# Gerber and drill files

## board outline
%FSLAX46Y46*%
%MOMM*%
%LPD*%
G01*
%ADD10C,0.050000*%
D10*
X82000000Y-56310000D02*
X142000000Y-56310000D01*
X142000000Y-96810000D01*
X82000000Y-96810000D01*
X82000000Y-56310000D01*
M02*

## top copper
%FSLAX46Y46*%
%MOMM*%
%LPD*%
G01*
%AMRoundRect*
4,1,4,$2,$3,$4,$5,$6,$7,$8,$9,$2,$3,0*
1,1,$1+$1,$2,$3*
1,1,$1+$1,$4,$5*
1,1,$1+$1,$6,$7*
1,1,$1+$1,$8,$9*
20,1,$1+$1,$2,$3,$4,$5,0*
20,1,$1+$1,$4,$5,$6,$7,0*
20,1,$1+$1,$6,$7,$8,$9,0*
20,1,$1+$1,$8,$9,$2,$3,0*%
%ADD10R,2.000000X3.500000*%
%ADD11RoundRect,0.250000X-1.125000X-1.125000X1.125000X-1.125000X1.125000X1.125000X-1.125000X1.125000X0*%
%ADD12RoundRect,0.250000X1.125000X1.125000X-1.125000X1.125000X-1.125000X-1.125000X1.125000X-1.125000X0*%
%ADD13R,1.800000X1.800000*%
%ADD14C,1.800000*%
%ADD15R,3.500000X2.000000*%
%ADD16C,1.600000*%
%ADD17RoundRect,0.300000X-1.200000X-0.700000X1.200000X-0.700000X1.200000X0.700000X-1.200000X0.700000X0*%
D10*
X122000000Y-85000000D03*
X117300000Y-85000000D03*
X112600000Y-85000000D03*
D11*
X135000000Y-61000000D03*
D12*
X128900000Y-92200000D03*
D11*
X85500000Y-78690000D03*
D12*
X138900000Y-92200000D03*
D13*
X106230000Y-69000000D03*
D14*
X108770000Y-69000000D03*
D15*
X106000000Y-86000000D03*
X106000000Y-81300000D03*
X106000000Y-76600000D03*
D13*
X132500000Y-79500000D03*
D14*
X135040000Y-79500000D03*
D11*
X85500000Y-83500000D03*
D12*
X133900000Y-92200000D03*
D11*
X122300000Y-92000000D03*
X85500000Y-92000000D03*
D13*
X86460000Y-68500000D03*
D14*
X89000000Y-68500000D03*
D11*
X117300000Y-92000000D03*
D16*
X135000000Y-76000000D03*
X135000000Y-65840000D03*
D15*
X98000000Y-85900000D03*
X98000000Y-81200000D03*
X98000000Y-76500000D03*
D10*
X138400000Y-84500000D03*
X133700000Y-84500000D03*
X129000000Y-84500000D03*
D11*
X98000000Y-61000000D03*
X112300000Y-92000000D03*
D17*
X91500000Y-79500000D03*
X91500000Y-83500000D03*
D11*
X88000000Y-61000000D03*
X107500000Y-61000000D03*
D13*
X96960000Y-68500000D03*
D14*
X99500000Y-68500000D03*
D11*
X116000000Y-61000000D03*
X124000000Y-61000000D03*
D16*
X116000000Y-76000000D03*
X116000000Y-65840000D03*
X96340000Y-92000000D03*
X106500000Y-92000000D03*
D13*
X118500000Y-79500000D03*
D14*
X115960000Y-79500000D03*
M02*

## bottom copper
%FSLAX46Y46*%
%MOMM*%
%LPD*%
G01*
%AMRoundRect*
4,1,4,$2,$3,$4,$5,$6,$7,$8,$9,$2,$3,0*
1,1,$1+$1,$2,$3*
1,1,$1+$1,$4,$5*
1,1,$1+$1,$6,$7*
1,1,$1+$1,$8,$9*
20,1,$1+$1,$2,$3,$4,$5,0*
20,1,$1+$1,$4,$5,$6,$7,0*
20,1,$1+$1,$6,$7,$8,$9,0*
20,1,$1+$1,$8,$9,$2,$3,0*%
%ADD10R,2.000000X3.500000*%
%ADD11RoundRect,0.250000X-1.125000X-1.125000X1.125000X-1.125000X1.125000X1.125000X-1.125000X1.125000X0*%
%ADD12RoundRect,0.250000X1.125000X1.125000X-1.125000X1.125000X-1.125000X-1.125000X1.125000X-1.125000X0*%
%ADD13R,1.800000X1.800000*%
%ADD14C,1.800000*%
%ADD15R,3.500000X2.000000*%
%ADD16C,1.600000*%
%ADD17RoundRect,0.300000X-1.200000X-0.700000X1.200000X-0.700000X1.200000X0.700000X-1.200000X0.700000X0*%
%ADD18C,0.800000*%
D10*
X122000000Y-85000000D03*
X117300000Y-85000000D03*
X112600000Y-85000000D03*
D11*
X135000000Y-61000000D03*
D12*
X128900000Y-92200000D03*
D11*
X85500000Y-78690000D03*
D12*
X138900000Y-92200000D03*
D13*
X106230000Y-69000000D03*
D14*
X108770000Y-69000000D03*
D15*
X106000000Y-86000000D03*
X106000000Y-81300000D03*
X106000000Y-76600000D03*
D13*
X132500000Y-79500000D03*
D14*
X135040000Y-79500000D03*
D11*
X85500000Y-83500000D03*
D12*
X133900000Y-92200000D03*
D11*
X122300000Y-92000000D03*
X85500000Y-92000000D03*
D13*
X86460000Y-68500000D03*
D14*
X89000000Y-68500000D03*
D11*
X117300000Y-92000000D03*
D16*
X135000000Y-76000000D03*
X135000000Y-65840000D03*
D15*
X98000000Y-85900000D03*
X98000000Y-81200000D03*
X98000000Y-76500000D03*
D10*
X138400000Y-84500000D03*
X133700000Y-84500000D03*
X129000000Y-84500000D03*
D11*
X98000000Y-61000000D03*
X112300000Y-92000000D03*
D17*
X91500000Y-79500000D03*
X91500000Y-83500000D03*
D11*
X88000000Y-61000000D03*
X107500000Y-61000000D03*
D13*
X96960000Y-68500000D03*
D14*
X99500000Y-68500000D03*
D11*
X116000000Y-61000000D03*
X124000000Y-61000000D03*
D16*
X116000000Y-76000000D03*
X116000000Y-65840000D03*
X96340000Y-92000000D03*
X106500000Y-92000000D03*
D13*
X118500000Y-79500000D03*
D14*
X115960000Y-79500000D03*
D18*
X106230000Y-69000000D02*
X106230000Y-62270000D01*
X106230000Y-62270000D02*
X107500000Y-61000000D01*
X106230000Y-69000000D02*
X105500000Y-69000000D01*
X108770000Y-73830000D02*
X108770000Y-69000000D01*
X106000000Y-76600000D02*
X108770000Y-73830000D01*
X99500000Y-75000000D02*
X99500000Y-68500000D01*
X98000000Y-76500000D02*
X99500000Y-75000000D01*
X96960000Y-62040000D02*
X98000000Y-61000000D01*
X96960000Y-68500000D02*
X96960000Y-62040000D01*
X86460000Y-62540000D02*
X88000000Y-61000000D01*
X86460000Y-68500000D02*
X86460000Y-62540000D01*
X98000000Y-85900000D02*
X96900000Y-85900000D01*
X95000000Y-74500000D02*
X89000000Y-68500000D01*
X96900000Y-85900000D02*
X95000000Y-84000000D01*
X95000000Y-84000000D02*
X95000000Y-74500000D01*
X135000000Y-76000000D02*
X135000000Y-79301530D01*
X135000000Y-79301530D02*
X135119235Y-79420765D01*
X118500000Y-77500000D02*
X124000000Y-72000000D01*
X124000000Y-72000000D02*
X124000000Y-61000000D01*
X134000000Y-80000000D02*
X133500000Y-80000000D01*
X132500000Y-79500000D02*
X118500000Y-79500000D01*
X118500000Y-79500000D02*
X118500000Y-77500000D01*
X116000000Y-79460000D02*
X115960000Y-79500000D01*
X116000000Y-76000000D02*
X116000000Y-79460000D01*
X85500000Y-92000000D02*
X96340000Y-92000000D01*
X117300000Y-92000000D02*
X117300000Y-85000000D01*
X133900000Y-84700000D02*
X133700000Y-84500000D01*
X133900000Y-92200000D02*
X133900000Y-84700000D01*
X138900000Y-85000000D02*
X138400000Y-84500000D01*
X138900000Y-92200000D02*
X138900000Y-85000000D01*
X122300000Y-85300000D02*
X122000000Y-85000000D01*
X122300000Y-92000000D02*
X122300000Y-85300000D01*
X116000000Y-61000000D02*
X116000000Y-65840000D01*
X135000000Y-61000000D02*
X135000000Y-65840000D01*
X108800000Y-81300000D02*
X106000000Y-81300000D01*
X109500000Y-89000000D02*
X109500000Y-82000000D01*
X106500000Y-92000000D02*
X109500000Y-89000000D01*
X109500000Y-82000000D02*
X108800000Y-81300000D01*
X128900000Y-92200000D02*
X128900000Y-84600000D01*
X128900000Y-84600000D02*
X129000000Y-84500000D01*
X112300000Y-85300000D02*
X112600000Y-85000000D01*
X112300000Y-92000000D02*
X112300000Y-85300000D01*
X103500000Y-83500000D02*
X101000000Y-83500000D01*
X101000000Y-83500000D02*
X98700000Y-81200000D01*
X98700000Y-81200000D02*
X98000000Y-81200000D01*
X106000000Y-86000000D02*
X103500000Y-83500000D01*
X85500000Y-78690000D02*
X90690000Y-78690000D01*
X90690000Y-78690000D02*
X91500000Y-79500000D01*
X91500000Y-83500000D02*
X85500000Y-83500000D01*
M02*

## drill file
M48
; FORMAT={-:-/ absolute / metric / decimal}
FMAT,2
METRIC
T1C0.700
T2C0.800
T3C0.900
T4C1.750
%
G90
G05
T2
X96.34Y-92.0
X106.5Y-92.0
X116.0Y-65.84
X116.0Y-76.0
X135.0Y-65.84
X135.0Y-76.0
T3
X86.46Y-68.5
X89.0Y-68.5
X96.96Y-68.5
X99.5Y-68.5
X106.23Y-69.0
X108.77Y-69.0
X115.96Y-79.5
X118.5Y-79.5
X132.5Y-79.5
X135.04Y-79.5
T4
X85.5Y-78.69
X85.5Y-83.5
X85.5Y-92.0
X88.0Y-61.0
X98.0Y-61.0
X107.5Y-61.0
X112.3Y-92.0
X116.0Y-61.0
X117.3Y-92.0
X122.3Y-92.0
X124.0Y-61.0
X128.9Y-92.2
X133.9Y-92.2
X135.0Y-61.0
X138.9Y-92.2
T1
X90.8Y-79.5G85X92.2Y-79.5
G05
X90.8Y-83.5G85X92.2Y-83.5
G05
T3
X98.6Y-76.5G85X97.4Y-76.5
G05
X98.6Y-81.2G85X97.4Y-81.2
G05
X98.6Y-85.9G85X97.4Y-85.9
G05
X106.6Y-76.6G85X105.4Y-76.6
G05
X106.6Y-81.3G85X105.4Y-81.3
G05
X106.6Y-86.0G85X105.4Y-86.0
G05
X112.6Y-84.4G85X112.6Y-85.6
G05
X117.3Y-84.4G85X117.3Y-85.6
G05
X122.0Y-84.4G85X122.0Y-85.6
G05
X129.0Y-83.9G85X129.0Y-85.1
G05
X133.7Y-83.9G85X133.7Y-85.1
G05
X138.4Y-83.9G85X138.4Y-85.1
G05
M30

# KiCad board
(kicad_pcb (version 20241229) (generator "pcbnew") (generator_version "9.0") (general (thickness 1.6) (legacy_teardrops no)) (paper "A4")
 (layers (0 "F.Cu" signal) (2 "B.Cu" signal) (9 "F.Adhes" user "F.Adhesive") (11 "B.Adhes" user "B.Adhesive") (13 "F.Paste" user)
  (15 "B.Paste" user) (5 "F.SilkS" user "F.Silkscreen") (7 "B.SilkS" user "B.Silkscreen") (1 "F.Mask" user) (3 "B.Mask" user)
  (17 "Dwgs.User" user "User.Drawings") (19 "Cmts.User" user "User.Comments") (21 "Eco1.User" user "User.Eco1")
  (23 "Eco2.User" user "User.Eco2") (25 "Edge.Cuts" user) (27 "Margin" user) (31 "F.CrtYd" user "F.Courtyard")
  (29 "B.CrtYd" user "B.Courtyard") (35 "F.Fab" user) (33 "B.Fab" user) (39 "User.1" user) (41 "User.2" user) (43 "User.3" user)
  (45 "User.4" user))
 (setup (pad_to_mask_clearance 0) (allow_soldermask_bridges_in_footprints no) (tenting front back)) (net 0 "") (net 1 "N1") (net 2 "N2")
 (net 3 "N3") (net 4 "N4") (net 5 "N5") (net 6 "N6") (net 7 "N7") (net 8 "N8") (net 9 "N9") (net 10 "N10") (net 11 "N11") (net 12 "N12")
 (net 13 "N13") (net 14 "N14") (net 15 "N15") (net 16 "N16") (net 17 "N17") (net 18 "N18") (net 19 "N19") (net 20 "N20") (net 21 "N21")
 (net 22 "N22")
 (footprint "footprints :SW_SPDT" (layer "F.Cu") (at 117.3 85 -90)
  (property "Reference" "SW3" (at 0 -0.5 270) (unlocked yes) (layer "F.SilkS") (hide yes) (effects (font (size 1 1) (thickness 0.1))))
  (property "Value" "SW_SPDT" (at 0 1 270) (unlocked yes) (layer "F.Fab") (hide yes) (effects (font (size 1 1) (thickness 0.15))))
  (pad "1" thru_hole rect (at 0 -4.7 270) (size 3.5 2) (drill oval 2.1 0.9) (layers "*.Cu" "*.Mask") (remove_unused_layers no) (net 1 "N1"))
  (pad "2" thru_hole rect (at 0 0 270) (size 3.5 2) (drill oval 2.1 0.9) (layers "*.Cu" "*.Mask") (remove_unused_layers no) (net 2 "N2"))
  (pad "3" thru_hole rect (at 0 4.7 270) (size 3.5 2) (drill oval 2.1 0.9) (layers "*.Cu" "*.Mask") (remove_unused_layers no) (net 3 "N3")))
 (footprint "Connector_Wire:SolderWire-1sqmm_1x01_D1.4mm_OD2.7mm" (layer "F.Cu") (at 135 61)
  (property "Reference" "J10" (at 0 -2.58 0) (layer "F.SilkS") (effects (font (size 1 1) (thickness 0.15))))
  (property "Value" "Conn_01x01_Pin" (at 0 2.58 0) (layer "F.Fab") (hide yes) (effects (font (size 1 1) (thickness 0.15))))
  (pad "1" thru_hole roundrect (at 0 0) (size 2.75 2.75) (drill 1.75) (layers "*.Cu" "*.Mask") (remove_unused_layers no)
   (roundrect_rratio 0.090909) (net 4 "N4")))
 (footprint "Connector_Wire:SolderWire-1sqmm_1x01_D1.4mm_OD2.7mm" (layer "F.Cu") (at 128.9 92.2 180)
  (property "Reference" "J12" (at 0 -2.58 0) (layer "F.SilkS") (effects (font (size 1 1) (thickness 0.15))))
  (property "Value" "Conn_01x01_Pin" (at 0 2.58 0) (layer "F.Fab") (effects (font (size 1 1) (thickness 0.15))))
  (pad "1" thru_hole roundrect (at 0 0 180) (size 2.75 2.75) (drill 1.75) (layers "*.Cu" "*.Mask") (remove_unused_layers no)
   (roundrect_rratio 0.090909) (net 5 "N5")))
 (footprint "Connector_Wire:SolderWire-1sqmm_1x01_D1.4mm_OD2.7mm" (layer "F.Cu") (at 85.5 78.69)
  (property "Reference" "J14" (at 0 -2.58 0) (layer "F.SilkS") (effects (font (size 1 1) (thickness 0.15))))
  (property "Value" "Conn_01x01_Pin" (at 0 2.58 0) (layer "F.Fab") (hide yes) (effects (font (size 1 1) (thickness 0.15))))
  (pad "1" thru_hole roundrect (at 0 0) (size 2.75 2.75) (drill 1.75) (layers "*.Cu" "*.Mask") (remove_unused_layers no)
   (roundrect_rratio 0.090909) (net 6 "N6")))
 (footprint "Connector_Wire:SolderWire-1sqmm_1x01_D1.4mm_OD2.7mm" (layer "F.Cu") (at 138.9 92.2 180)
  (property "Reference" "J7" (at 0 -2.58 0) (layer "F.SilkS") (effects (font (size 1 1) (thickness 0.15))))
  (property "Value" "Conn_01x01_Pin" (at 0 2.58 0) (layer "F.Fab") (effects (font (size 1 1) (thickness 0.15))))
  (pad "1" thru_hole roundrect (at 0 0 180) (size 2.75 2.75) (drill 1.75) (layers "*.Cu" "*.Mask") (remove_unused_layers no)
   (roundrect_rratio 0.090909) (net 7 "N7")))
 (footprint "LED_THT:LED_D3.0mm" (layer "F.Cu") (at 106.23 69)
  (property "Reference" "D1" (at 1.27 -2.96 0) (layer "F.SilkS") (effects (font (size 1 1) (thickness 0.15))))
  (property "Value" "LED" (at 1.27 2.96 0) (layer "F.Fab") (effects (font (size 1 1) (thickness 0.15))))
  (pad "1" thru_hole rect (at 0 0) (size 1.8 1.8) (drill 0.9) (layers "*.Cu" "*.Mask") (remove_unused_layers no) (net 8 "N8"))
  (pad "2" thru_hole circle (at 2.54 0) (size 1.8 1.8) (drill 0.9) (layers "*.Cu" "*.Mask") (remove_unused_layers no) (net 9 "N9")))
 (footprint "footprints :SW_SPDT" (layer "F.Cu") (at 106 81.3 180)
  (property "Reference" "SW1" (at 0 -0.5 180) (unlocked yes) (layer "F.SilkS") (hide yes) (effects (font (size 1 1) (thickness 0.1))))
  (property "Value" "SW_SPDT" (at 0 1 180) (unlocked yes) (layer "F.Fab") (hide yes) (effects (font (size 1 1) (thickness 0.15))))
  (pad "1" thru_hole rect (at 0 -4.7 180) (size 3.5 2) (drill oval 2.1 0.9) (layers "*.Cu" "*.Mask") (remove_unused_layers no)
   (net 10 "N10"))
  (pad "2" thru_hole rect (at 0 0 180) (size 3.5 2) (drill oval 2.1 0.9) (layers "*.Cu" "*.Mask") (remove_unused_layers no) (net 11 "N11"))
  (pad "3" thru_hole rect (at 0 4.7 180) (size 3.5 2) (drill oval 2.1 0.9) (layers "*.Cu" "*.Mask") (remove_unused_layers no) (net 9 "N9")))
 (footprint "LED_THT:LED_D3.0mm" (layer "F.Cu") (at 132.5 79.5)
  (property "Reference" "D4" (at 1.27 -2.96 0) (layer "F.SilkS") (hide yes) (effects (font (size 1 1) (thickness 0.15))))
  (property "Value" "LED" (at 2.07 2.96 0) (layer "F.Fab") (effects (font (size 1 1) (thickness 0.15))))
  (pad "1" thru_hole rect (at 0 0) (size 1.8 1.8) (drill 0.9) (layers "*.Cu" "*.Mask") (remove_unused_layers no) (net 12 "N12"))
  (pad "2" thru_hole circle (at 2.54 0) (size 1.8 1.8) (drill 0.9) (layers "*.Cu" "*.Mask") (remove_unused_layers no) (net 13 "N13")))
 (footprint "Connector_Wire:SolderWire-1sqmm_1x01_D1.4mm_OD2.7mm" (layer "F.Cu") (at 85.5 83.5)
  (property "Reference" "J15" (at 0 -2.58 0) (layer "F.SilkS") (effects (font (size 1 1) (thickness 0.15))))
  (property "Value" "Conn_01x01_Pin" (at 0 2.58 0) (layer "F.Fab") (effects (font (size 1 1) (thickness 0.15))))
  (pad "1" thru_hole roundrect (at 0 0) (size 2.75 2.75) (drill 1.75) (layers "*.Cu" "*.Mask") (remove_unused_layers no)
   (roundrect_rratio 0.090909) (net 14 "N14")))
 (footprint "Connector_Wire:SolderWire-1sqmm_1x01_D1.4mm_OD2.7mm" (layer "F.Cu") (at 133.9 92.2 180)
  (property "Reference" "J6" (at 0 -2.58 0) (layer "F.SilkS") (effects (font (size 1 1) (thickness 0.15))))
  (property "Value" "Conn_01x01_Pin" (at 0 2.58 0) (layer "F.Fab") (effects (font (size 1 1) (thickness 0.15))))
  (pad "1" thru_hole roundrect (at 0 0 180) (size 2.75 2.75) (drill 1.75) (layers "*.Cu" "*.Mask") (remove_unused_layers no)
   (roundrect_rratio 0.090909) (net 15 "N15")))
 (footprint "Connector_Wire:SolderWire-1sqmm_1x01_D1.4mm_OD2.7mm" (layer "F.Cu") (at 122.3 92)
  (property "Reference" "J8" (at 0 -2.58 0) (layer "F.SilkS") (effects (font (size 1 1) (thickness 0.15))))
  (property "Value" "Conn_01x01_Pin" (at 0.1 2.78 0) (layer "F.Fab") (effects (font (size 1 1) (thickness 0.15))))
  (pad "1" thru_hole roundrect (at 0 0) (size 2.75 2.75) (drill 1.75) (layers "*.Cu" "*.Mask") (remove_unused_layers no)
   (roundrect_rratio 0.090909) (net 1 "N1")))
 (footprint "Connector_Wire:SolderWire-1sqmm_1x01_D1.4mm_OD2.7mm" (layer "F.Cu") (at 85.5 92)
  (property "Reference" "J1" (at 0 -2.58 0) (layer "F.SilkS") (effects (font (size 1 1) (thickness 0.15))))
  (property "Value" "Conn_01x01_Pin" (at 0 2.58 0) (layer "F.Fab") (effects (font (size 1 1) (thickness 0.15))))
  (pad "1" thru_hole roundrect (at 0 0) (size 2.75 2.75) (drill 1.75) (layers "*.Cu" "*.Mask") (remove_unused_layers no)
   (roundrect_rratio 0.090909) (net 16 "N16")))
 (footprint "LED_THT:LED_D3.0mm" (layer "F.Cu") (at 86.46 68.5)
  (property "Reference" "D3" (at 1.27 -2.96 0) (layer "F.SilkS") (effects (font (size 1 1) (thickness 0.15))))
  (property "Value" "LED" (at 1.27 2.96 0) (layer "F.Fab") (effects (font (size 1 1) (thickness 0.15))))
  (pad "1" thru_hole rect (at 0 0) (size 1.8 1.8) (drill 0.9) (layers "*.Cu" "*.Mask") (remove_unused_layers no) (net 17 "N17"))
  (pad "2" thru_hole circle (at 2.54 0) (size 1.8 1.8) (drill 0.9) (layers "*.Cu" "*.Mask") (remove_unused_layers no) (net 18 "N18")))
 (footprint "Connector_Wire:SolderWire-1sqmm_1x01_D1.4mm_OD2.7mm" (layer "F.Cu") (at 117.3 92)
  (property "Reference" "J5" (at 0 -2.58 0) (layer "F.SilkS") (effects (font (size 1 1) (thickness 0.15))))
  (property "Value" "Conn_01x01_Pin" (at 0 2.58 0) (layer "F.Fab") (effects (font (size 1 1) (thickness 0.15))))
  (pad "1" thru_hole roundrect (at 0 0) (size 2.75 2.75) (drill 1.75) (layers "*.Cu" "*.Mask") (remove_unused_layers no)
   (roundrect_rratio 0.090909) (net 2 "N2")))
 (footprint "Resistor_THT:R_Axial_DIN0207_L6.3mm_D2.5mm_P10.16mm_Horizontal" (layer "F.Cu") (at 135 76 90)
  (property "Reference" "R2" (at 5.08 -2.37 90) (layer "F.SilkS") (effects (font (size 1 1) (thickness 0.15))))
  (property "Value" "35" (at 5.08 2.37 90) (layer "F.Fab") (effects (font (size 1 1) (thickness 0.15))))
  (pad "1" thru_hole circle (at 0 0 90) (size 1.6 1.6) (drill 0.8) (layers "*.Cu" "*.Mask") (remove_unused_layers no) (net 13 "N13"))
  (pad "2" thru_hole circle (at 10.16 0 90) (size 1.6 1.6) (drill 0.8) (layers "*.Cu" "*.Mask") (remove_unused_layers no) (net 4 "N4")))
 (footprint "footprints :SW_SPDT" (layer "F.Cu") (at 98 81.2 180)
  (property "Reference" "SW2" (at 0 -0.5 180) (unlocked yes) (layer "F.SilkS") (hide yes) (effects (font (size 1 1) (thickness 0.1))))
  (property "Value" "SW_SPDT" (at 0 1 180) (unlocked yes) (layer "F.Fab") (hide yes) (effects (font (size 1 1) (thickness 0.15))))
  (pad "1" thru_hole rect (at 0 -4.7 180) (size 3.5 2) (drill oval 2.1 0.9) (layers "*.Cu" "*.Mask") (remove_unused_layers no)
   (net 18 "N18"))
  (pad "2" thru_hole rect (at 0 0 180) (size 3.5 2) (drill oval 2.1 0.9) (layers "*.Cu" "*.Mask") (remove_unused_layers no) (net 10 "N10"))
  (pad "3" thru_hole rect (at 0 4.7 180) (size 3.5 2) (drill oval 2.1 0.9) (layers "*.Cu" "*.Mask") (remove_unused_layers no) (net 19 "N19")))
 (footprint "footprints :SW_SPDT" (layer "F.Cu") (at 133.7 84.5 -90)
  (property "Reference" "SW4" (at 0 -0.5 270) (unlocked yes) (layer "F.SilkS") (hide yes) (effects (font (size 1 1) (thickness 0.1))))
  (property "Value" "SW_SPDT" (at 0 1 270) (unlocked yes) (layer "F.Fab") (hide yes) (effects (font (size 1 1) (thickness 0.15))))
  (pad "1" thru_hole rect (at 0 -4.7 270) (size 3.5 2) (drill oval 2.1 0.9) (layers "*.Cu" "*.Mask") (remove_unused_layers no) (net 7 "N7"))
  (pad "2" thru_hole rect (at 0 0 270) (size 3.5 2) (drill oval 2.1 0.9) (layers "*.Cu" "*.Mask") (remove_unused_layers no) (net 15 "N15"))
  (pad "3" thru_hole rect (at 0 4.7 270) (size 3.5 2) (drill oval 2.1 0.9) (layers "*.Cu" "*.Mask") (remove_unused_layers no) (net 5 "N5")))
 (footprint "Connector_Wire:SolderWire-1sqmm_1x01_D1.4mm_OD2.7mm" (layer "F.Cu") (at 98 61)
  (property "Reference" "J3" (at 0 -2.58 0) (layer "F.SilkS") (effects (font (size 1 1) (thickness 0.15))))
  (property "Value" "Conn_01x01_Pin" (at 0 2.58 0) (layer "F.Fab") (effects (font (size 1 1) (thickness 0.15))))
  (pad "1" thru_hole roundrect (at 0 0) (size 2.75 2.75) (drill 1.75) (layers "*.Cu" "*.Mask") (remove_unused_layers no)
   (roundrect_rratio 0.090909) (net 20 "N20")))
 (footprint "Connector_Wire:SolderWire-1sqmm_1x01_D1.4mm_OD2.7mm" (layer "F.Cu") (at 112.3 92)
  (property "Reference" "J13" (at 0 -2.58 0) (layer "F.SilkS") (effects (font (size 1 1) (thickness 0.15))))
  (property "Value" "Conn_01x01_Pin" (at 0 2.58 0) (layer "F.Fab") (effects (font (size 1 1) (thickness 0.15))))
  (pad "1" thru_hole roundrect (at 0 0) (size 2.75 2.75) (drill 1.75) (layers "*.Cu" "*.Mask") (remove_unused_layers no)
   (roundrect_rratio 0.090909) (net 3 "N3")))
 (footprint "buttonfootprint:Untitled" (layer "F.Cu") (at 91.5 79.5)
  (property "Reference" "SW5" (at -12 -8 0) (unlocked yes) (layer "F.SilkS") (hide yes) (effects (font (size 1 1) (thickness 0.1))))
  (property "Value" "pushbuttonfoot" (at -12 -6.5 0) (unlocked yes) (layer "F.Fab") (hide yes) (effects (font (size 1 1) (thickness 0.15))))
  (pad "1" thru_hole roundrect (at 0 0) (size 3 2) (drill oval 2.1 0.7) (layers "*.Cu" "*.Mask") (remove_unused_layers no)
   (roundrect_rratio 0.15) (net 6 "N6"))
  (pad "2" thru_hole roundrect (at 0 4) (size 3 2) (drill oval 2.1 0.7) (layers "*.Cu" "*.Mask") (remove_unused_layers no)
   (roundrect_rratio 0.15) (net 14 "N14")))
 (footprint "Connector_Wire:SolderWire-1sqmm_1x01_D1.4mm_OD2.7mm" (layer "F.Cu") (at 88 61)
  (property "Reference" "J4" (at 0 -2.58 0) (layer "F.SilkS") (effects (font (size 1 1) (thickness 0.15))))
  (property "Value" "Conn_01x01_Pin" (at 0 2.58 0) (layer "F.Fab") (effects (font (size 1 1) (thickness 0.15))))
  (pad "1" thru_hole roundrect (at 0 0) (size 2.75 2.75) (drill 1.75) (layers "*.Cu" "*.Mask") (remove_unused_layers no)
   (roundrect_rratio 0.090909) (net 17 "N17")))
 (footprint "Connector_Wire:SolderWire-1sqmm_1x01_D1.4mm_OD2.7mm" (layer "F.Cu") (at 107.5 61)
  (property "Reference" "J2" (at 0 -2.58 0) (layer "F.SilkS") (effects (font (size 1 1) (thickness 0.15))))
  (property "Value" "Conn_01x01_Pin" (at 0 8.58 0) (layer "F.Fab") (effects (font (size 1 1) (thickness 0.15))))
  (pad "1" thru_hole roundrect (at 0 0) (size 2.75 2.75) (drill 1.75) (layers "*.Cu" "*.Mask") (remove_unused_layers no)
   (roundrect_rratio 0.090909) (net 8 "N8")))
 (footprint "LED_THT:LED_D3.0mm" (layer "F.Cu") (at 96.96 68.5)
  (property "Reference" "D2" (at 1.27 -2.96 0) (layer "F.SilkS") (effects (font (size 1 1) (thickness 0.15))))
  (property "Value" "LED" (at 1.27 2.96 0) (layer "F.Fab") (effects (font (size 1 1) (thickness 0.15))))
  (pad "1" thru_hole rect (at 0 0) (size 1.8 1.8) (drill 0.9) (layers "*.Cu" "*.Mask") (remove_unused_layers no) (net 20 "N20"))
  (pad "2" thru_hole circle (at 2.54 0) (size 1.8 1.8) (drill 0.9) (layers "*.Cu" "*.Mask") (remove_unused_layers no) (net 19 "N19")))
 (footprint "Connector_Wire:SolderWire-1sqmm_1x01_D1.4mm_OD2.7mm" (layer "F.Cu") (at 116 61)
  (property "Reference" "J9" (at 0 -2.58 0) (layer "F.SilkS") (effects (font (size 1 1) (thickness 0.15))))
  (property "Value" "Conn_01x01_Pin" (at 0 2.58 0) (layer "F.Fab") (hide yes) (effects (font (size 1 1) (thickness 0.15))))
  (pad "1" thru_hole roundrect (at 0 0) (size 2.75 2.75) (drill 1.75) (layers "*.Cu" "*.Mask") (remove_unused_layers no)
   (roundrect_rratio 0.090909) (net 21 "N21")))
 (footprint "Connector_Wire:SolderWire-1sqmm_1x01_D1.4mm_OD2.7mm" (layer "F.Cu") (at 124 61)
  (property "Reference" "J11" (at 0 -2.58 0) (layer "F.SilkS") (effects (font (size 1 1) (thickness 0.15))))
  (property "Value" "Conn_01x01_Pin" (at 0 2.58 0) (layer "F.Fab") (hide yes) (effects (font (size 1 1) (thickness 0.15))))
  (pad "1" thru_hole roundrect (at 0 0) (size 2.75 2.75) (drill 1.75) (layers "*.Cu" "*.Mask") (remove_unused_layers no)
   (roundrect_rratio 0.090909) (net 12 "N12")))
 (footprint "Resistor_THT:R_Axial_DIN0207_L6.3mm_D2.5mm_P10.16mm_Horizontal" (layer "F.Cu") (at 116 76 90)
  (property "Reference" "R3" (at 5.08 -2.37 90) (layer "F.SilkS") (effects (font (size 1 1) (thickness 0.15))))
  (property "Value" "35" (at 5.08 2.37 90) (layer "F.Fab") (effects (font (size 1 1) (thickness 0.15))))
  (pad "1" thru_hole circle (at 0 0 90) (size 1.6 1.6) (drill 0.8) (layers "*.Cu" "*.Mask") (remove_unused_layers no) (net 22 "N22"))
  (pad "2" thru_hole circle (at 10.16 0 90) (size 1.6 1.6) (drill 0.8) (layers "*.Cu" "*.Mask") (remove_unused_layers no) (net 21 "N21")))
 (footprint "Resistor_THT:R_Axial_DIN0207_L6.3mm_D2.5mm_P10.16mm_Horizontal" (layer "F.Cu") (at 96.34 92)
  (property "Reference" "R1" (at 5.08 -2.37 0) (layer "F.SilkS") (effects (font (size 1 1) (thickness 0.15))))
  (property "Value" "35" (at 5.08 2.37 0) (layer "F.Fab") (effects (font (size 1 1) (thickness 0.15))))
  (pad "1" thru_hole circle (at 0 0) (size 1.6 1.6) (drill 0.8) (layers "*.Cu" "*.Mask") (remove_unused_layers no) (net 16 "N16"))
  (pad "2" thru_hole circle (at 10.16 0) (size 1.6 1.6) (drill 0.8) (layers "*.Cu" "*.Mask") (remove_unused_layers no) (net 11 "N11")))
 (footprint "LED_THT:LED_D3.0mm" (layer "F.Cu") (at 118.5 79.5 180)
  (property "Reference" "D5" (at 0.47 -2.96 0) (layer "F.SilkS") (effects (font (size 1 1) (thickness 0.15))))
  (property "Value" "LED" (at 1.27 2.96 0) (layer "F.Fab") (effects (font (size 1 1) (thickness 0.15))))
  (pad "1" thru_hole rect (at 0 0 180) (size 1.8 1.8) (drill 0.9) (layers "*.Cu" "*.Mask") (remove_unused_layers no) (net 12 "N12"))
  (pad "2" thru_hole circle (at 2.54 0 180) (size 1.8 1.8) (drill 0.9) (layers "*.Cu" "*.Mask") (remove_unused_layers no) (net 22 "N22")))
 (gr_rect (start 82 56.31) (end 142 96.81) (stroke (width 0.05) (type solid)) (fill no) (layer "Edge.Cuts"))
 (segment (start 106.23 69) (end 106.23 62.27) (width 0.8) (layer "B.Cu") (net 8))
 (segment (start 106.23 62.27) (end 107.5 61) (width 0.8) (layer "B.Cu") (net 8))
 (segment (start 106.23 69) (end 105.5 69) (width 0.8) (layer "B.Cu") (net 8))
 (segment (start 108.77 73.83) (end 108.77 69) (width 0.8) (layer "B.Cu") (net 9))
 (segment (start 106 76.6) (end 108.77 73.83) (width 0.8) (layer "B.Cu") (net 9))
 (segment (start 99.5 75) (end 99.5 68.5) (width 0.8) (layer "B.Cu") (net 19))
 (segment (start 98 76.5) (end 99.5 75) (width 0.8) (layer "B.Cu") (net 19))
 (segment (start 96.96 62.04) (end 98 61) (width 0.8) (layer "B.Cu") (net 20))
 (segment (start 96.96 68.5) (end 96.96 62.04) (width 0.8) (layer "B.Cu") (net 20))
 (segment (start 86.46 62.54) (end 88 61) (width 0.8) (layer "B.Cu") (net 17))
 (segment (start 86.46 68.5) (end 86.46 62.54) (width 0.8) (layer "B.Cu") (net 17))
 (segment (start 98 85.9) (end 96.9 85.9) (width 0.8) (layer "B.Cu") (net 18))
 (segment (start 95 74.5) (end 89 68.5) (width 0.8) (layer "B.Cu") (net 18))
 (segment (start 96.9 85.9) (end 95 84) (width 0.8) (layer "B.Cu") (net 18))
 (segment (start 95 84) (end 95 74.5) (width 0.8) (layer "B.Cu") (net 18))
 (segment (start 135 76) (end 135 79.30153) (width 0.8) (layer "B.Cu") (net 13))
 (segment (start 135 79.30153) (end 135.119235 79.420765) (width 0.8) (layer "B.Cu") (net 13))
 (segment (start 118.5 77.5) (end 124 72) (width 0.8) (layer "B.Cu") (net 12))
 (segment (start 124 72) (end 124 61) (width 0.8) (layer "B.Cu") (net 12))
 (segment (start 134 80) (end 133.5 80) (width 0.8) (layer "B.Cu") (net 12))
 (segment (start 132.5 79.5) (end 118.5 79.5) (width 0.8) (layer "B.Cu") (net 12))
 (segment (start 118.5 79.5) (end 118.5 77.5) (width 0.8) (layer "B.Cu") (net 12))
 (segment (start 116 79.46) (end 115.96 79.5) (width 0.8) (layer "B.Cu") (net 22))
 (segment (start 116 76) (end 116 79.46) (width 0.8) (layer "B.Cu") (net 22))
 (segment (start 85.5 92) (end 96.34 92) (width 0.8) (layer "B.Cu") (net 16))
 (segment (start 117.3 92) (end 117.3 85) (width 0.8) (layer "B.Cu") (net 2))
 (segment (start 133.9 84.7) (end 133.7 84.5) (width 0.8) (layer "B.Cu") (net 15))
 (segment (start 133.9 92.2) (end 133.9 84.7) (width 0.8) (layer "B.Cu") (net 15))
 (segment (start 138.9 85) (end 138.4 84.5) (width 0.8) (layer "B.Cu") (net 7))
 (segment (start 138.9 92.2) (end 138.9 85) (width 0.8) (layer "B.Cu") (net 7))
 (segment (start 122.3 85.3) (end 122 85) (width 0.8) (layer "B.Cu") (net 1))
 (segment (start 122.3 92) (end 122.3 85.3) (width 0.8) (layer "B.Cu") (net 1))
 (segment (start 116 61) (end 116 65.84) (width 0.8) (layer "B.Cu") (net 21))
 (segment (start 135 61) (end 135 65.84) (width 0.8) (layer "B.Cu") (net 4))
 (segment (start 108.8 81.3) (end 106 81.3) (width 0.8) (layer "B.Cu") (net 11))
 (segment (start 109.5 89) (end 109.5 82) (width 0.8) (layer "B.Cu") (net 11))
 (segment (start 106.5 92) (end 109.5 89) (width 0.8) (layer "B.Cu") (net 11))
 (segment (start 109.5 82) (end 108.8 81.3) (width 0.8) (layer "B.Cu") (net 11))
 (segment (start 128.9 92.2) (end 128.9 84.6) (width 0.8) (layer "B.Cu") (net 5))
 (segment (start 128.9 84.6) (end 129 84.5) (width 0.8) (layer "B.Cu") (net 5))
 (segment (start 112.3 85.3) (end 112.6 85) (width 0.8) (layer "B.Cu") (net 3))
 (segment (start 112.3 92) (end 112.3 85.3) (width 0.8) (layer "B.Cu") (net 3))
 (segment (start 103.5 83.5) (end 101 83.5) (width 0.8) (layer "B.Cu") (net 10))
 (segment (start 101 83.5) (end 98.7 81.2) (width 0.8) (layer "B.Cu") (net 10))
 (segment (start 98.7 81.2) (end 98 81.2) (width 0.8) (layer "B.Cu") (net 10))
 (segment (start 106 86) (end 103.5 83.5) (width 0.8) (layer "B.Cu") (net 10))
 (segment (start 85.5 78.69) (end 90.69 78.69) (width 0.8) (layer "B.Cu") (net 6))
 (segment (start 90.69 78.69) (end 91.5 79.5) (width 0.8) (layer "B.Cu") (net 6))
 (segment (start 91.5 83.5) (end 85.5 83.5) (width 0.8) (layer "B.Cu") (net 14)))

